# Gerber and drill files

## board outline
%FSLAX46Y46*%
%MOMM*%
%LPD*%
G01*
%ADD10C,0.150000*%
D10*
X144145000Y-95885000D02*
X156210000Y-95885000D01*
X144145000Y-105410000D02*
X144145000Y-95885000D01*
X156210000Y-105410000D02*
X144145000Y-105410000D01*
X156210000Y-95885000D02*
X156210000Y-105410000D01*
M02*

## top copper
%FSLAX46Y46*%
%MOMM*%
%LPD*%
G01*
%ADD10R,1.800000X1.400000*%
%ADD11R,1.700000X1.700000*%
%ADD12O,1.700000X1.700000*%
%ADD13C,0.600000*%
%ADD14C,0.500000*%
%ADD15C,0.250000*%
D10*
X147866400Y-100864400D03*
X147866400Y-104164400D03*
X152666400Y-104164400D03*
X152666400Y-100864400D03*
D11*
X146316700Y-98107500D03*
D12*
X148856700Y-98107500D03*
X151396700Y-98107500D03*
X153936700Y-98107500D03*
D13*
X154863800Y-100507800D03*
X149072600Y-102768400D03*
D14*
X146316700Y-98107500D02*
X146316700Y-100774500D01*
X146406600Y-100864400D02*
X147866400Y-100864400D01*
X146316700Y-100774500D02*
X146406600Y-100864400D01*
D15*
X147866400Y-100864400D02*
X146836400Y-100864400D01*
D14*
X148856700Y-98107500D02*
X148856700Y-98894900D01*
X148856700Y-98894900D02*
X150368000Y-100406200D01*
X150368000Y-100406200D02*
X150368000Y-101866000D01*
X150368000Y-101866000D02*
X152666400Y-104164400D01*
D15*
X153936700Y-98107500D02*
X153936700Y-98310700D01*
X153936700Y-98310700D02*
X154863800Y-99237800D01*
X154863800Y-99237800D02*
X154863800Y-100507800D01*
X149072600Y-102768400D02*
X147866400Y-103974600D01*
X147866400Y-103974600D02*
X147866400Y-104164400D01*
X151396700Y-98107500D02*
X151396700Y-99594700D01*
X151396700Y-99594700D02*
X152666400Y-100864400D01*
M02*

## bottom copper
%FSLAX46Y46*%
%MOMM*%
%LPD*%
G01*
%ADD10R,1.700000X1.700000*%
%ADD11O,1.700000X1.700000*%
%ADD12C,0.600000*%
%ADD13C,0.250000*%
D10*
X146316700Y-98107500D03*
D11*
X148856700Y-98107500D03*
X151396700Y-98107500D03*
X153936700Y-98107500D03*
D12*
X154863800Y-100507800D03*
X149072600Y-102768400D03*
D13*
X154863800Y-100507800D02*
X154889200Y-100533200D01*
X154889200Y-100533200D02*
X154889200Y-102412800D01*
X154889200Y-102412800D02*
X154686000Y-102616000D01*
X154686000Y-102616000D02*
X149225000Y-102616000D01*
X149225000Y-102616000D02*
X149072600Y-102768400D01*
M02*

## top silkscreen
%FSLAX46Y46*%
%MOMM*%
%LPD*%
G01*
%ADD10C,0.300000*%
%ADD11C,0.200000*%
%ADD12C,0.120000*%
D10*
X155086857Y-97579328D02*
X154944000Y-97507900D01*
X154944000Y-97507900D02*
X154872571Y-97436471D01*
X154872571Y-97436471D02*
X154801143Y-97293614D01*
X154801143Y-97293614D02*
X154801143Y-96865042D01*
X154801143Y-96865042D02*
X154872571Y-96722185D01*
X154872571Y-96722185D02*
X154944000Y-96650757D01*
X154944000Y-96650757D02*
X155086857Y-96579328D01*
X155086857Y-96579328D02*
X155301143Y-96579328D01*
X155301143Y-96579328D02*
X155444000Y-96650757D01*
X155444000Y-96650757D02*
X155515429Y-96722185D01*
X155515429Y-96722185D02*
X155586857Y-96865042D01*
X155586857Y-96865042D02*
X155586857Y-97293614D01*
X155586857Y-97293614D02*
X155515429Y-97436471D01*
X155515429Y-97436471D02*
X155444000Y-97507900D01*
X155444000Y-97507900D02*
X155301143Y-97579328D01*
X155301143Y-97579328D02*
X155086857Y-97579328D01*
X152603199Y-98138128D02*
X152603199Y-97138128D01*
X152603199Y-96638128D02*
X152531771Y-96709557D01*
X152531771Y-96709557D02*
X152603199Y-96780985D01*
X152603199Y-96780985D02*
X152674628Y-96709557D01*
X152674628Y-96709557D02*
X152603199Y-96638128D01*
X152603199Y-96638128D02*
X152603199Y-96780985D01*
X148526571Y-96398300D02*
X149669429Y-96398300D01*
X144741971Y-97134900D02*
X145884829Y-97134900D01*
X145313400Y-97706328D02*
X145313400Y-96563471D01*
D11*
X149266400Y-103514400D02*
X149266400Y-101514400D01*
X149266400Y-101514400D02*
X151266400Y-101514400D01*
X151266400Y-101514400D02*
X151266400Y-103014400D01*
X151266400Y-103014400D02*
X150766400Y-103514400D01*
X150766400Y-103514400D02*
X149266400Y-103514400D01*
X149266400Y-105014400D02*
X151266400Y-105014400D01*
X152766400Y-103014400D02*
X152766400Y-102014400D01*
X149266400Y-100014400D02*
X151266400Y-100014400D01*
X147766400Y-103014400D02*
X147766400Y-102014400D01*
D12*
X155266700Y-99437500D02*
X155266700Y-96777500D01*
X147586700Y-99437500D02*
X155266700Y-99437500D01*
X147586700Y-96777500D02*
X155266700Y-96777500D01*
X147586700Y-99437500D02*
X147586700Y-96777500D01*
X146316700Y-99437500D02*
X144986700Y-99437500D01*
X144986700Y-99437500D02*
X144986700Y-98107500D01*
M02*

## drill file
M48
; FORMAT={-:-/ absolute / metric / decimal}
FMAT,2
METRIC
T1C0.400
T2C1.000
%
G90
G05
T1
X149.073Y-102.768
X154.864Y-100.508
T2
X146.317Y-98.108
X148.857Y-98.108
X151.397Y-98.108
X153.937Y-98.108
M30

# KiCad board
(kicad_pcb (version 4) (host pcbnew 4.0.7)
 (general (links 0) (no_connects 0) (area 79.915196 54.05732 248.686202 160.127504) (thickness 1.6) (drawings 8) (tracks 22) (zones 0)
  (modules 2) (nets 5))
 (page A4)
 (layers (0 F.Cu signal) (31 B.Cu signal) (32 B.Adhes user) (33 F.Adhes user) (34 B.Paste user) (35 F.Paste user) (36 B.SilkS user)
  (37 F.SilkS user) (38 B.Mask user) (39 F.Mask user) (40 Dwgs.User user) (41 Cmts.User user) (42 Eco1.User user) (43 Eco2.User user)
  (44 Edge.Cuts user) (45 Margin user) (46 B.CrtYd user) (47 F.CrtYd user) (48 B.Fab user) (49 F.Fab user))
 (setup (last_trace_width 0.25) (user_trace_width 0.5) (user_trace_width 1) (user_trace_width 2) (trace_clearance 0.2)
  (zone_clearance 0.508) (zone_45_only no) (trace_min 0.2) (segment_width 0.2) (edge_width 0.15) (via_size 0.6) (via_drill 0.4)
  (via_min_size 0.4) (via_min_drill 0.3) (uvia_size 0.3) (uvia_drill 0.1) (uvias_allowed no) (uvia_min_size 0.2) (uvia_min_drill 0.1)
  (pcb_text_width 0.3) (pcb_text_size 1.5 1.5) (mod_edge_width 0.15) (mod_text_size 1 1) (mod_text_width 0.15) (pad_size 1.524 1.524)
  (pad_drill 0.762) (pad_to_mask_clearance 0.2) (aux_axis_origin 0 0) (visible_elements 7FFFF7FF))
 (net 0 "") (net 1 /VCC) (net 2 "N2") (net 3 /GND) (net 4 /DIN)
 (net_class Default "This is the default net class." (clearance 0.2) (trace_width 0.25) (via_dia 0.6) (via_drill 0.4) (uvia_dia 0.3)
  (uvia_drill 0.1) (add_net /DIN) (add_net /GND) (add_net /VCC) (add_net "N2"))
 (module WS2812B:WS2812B (layer F.Cu) (at 150.2664 102.5144 90)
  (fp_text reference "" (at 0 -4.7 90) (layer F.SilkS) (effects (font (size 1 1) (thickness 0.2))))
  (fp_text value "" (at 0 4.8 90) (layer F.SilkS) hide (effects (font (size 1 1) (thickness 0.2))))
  (fp_line (start -1 -1) (end 1 -1) (layer F.SilkS) (width 0.2)) (fp_line (start 1 -1) (end 1 1) (layer F.SilkS) (width 0.2))
  (fp_line (start 1 1) (end -0.5 1) (layer F.SilkS) (width 0.2))
  (fp_line (start -0.5 1) (end -1 0.5) (layer F.SilkS) (width 0.2))
  (fp_line (start -1 0.5) (end -1 -1) (layer F.SilkS) (width 0.2))
  (fp_line (start -2.5 -1) (end -2.5 1) (layer F.SilkS) (width 0.2))
  (fp_line (start -0.5 2.5) (end 0.5 2.5) (layer F.SilkS) (width 0.2))
  (fp_line (start 2.5 -1) (end 2.5 1) (layer F.SilkS) (width 0.2))
  (fp_line (start -0.5 -2.5) (end 0.5 -2.5) (layer F.SilkS) (width 0.2))
  (pad 1 smd rect (at 1.65 -2.4 90) (size 1.4 1.8) (layers F.Cu F.Paste F.Mask) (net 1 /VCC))
  (pad 2 smd rect (at -1.65 -2.4 90) (size 1.4 1.8) (layers F.Cu F.Paste F.Mask) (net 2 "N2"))
  (pad 3 smd rect (at -1.65 2.4 90) (size 1.4 1.8) (layers F.Cu F.Paste F.Mask) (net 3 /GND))
  (pad 4 smd rect (at 1.65 2.4 90) (size 1.4 1.8) (layers F.Cu F.Paste F.Mask) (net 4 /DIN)))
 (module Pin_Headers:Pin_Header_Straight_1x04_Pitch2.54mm (layer F.Cu) (at 146.3167 98.1075 90)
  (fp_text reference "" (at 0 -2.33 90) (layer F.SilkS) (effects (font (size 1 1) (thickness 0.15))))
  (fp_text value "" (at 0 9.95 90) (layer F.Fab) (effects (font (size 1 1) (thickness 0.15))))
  (fp_line (start -1.33 8.95) (end 1.33 8.95) (layer F.SilkS) (width 0.12))
  (fp_line (start -1.33 1.27) (end -1.33 8.95) (layer F.SilkS) (width 0.12))
  (fp_line (start 1.33 1.27) (end 1.33 8.95) (layer F.SilkS) (width 0.12))
  (fp_line (start -1.33 1.27) (end 1.33 1.27) (layer F.SilkS) (width 0.12))
  (fp_line (start -1.33 0) (end -1.33 -1.33) (layer F.SilkS) (width 0.12))
  (fp_line (start -1.33 -1.33) (end 0 -1.33) (layer F.SilkS) (width 0.12))
  (pad 1 thru_hole rect (at 0 0 90) (size 1.7 1.7) (drill 1) (layers *.Cu *.Mask))
  (pad 2 thru_hole oval (at 0 2.54 90) (size 1.7 1.7) (drill 1) (layers *.Cu *.Mask))
  (pad 3 thru_hole oval (at 0 5.08 90) (size 1.7 1.7) (drill 1) (layers *.Cu *.Mask))
  (pad 4 thru_hole oval (at 0 7.62 90) (size 1.7 1.7) (drill 1) (layers *.Cu *.Mask)))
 (gr_line (start 144.145 95.885) (end 156.21 95.885) (angle 90) (layer Edge.Cuts) (width 0.15))
 (gr_line (start 144.145 105.41) (end 144.145 95.885) (angle 90) (layer Edge.Cuts) (width 0.15))
 (gr_line (start 156.21 105.41) (end 144.145 105.41) (angle 90) (layer Edge.Cuts) (width 0.15))
 (gr_line (start 156.21 95.885) (end 156.21 105.41) (angle 90) (layer Edge.Cuts) (width 0.15))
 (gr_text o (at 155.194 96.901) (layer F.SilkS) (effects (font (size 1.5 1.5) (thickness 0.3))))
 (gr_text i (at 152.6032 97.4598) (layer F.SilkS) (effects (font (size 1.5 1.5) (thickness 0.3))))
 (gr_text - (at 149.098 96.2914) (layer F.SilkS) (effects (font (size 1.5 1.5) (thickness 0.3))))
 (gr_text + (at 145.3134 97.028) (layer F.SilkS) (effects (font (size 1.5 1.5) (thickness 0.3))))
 (segment (start 146.3167 98.1075) (end 146.3167 100.7745) (width 0.5) (layer F.Cu) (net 1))
 (segment (start 146.4066 100.8644) (end 147.8664 100.8644) (width 0.5) (layer F.Cu) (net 1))
 (segment (start 146.3167 100.7745) (end 146.4066 100.8644) (width 0.5) (layer F.Cu) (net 1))
 (segment (start 147.8664 100.8644) (end 146.8364 100.8644) (width 0.25) (layer F.Cu) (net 1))
 (segment (start 148.8567 98.1075) (end 148.8567 98.8949) (width 0.5) (layer F.Cu) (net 3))
 (segment (start 148.8567 98.8949) (end 150.368 100.4062) (width 0.5) (layer F.Cu) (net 3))
 (segment (start 150.368 100.4062) (end 150.368 101.866) (width 0.5) (layer F.Cu) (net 3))
 (segment (start 150.368 101.866) (end 152.6664 104.1644) (width 0.5) (layer F.Cu) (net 3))
 (segment (start 153.9367 98.1075) (end 153.9367 98.3107) (width 0.25) (layer F.Cu) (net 2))
 (segment (start 153.9367 98.3107) (end 154.8638 99.2378) (width 0.25) (layer F.Cu) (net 2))
 (segment (start 154.8638 99.2378) (end 154.8638 100.5078) (width 0.25) (layer F.Cu) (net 2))
 (via (at 154.8638 100.5078) (size 0.6) (drill 0.4) (layers F.Cu B.Cu) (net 2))
 (segment (start 154.8638 100.5078) (end 154.8892 100.5332) (width 0.25) (layer B.Cu) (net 2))
 (segment (start 154.8892 100.5332) (end 154.8892 102.4128) (width 0.25) (layer B.Cu) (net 2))
 (segment (start 154.8892 102.4128) (end 154.686 102.616) (width 0.25) (layer B.Cu) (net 2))
 (segment (start 154.686 102.616) (end 149.225 102.616) (width 0.25) (layer B.Cu) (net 2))
 (segment (start 149.225 102.616) (end 149.0726 102.7684) (width 0.25) (layer B.Cu) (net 2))
 (via (at 149.0726 102.7684) (size 0.6) (drill 0.4) (layers F.Cu B.Cu) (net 2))
 (segment (start 149.0726 102.7684) (end 147.8664 103.9746) (width 0.25) (layer F.Cu) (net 2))
 (segment (start 147.8664 103.9746) (end 147.8664 104.1644) (width 0.25) (layer F.Cu) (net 2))
 (segment (start 151.3967 98.1075) (end 151.3967 99.5947) (width 0.25) (layer F.Cu) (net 4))
 (segment (start 151.3967 99.5947) (end 152.6664 100.8644) (width 0.25) (layer F.Cu) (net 4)))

